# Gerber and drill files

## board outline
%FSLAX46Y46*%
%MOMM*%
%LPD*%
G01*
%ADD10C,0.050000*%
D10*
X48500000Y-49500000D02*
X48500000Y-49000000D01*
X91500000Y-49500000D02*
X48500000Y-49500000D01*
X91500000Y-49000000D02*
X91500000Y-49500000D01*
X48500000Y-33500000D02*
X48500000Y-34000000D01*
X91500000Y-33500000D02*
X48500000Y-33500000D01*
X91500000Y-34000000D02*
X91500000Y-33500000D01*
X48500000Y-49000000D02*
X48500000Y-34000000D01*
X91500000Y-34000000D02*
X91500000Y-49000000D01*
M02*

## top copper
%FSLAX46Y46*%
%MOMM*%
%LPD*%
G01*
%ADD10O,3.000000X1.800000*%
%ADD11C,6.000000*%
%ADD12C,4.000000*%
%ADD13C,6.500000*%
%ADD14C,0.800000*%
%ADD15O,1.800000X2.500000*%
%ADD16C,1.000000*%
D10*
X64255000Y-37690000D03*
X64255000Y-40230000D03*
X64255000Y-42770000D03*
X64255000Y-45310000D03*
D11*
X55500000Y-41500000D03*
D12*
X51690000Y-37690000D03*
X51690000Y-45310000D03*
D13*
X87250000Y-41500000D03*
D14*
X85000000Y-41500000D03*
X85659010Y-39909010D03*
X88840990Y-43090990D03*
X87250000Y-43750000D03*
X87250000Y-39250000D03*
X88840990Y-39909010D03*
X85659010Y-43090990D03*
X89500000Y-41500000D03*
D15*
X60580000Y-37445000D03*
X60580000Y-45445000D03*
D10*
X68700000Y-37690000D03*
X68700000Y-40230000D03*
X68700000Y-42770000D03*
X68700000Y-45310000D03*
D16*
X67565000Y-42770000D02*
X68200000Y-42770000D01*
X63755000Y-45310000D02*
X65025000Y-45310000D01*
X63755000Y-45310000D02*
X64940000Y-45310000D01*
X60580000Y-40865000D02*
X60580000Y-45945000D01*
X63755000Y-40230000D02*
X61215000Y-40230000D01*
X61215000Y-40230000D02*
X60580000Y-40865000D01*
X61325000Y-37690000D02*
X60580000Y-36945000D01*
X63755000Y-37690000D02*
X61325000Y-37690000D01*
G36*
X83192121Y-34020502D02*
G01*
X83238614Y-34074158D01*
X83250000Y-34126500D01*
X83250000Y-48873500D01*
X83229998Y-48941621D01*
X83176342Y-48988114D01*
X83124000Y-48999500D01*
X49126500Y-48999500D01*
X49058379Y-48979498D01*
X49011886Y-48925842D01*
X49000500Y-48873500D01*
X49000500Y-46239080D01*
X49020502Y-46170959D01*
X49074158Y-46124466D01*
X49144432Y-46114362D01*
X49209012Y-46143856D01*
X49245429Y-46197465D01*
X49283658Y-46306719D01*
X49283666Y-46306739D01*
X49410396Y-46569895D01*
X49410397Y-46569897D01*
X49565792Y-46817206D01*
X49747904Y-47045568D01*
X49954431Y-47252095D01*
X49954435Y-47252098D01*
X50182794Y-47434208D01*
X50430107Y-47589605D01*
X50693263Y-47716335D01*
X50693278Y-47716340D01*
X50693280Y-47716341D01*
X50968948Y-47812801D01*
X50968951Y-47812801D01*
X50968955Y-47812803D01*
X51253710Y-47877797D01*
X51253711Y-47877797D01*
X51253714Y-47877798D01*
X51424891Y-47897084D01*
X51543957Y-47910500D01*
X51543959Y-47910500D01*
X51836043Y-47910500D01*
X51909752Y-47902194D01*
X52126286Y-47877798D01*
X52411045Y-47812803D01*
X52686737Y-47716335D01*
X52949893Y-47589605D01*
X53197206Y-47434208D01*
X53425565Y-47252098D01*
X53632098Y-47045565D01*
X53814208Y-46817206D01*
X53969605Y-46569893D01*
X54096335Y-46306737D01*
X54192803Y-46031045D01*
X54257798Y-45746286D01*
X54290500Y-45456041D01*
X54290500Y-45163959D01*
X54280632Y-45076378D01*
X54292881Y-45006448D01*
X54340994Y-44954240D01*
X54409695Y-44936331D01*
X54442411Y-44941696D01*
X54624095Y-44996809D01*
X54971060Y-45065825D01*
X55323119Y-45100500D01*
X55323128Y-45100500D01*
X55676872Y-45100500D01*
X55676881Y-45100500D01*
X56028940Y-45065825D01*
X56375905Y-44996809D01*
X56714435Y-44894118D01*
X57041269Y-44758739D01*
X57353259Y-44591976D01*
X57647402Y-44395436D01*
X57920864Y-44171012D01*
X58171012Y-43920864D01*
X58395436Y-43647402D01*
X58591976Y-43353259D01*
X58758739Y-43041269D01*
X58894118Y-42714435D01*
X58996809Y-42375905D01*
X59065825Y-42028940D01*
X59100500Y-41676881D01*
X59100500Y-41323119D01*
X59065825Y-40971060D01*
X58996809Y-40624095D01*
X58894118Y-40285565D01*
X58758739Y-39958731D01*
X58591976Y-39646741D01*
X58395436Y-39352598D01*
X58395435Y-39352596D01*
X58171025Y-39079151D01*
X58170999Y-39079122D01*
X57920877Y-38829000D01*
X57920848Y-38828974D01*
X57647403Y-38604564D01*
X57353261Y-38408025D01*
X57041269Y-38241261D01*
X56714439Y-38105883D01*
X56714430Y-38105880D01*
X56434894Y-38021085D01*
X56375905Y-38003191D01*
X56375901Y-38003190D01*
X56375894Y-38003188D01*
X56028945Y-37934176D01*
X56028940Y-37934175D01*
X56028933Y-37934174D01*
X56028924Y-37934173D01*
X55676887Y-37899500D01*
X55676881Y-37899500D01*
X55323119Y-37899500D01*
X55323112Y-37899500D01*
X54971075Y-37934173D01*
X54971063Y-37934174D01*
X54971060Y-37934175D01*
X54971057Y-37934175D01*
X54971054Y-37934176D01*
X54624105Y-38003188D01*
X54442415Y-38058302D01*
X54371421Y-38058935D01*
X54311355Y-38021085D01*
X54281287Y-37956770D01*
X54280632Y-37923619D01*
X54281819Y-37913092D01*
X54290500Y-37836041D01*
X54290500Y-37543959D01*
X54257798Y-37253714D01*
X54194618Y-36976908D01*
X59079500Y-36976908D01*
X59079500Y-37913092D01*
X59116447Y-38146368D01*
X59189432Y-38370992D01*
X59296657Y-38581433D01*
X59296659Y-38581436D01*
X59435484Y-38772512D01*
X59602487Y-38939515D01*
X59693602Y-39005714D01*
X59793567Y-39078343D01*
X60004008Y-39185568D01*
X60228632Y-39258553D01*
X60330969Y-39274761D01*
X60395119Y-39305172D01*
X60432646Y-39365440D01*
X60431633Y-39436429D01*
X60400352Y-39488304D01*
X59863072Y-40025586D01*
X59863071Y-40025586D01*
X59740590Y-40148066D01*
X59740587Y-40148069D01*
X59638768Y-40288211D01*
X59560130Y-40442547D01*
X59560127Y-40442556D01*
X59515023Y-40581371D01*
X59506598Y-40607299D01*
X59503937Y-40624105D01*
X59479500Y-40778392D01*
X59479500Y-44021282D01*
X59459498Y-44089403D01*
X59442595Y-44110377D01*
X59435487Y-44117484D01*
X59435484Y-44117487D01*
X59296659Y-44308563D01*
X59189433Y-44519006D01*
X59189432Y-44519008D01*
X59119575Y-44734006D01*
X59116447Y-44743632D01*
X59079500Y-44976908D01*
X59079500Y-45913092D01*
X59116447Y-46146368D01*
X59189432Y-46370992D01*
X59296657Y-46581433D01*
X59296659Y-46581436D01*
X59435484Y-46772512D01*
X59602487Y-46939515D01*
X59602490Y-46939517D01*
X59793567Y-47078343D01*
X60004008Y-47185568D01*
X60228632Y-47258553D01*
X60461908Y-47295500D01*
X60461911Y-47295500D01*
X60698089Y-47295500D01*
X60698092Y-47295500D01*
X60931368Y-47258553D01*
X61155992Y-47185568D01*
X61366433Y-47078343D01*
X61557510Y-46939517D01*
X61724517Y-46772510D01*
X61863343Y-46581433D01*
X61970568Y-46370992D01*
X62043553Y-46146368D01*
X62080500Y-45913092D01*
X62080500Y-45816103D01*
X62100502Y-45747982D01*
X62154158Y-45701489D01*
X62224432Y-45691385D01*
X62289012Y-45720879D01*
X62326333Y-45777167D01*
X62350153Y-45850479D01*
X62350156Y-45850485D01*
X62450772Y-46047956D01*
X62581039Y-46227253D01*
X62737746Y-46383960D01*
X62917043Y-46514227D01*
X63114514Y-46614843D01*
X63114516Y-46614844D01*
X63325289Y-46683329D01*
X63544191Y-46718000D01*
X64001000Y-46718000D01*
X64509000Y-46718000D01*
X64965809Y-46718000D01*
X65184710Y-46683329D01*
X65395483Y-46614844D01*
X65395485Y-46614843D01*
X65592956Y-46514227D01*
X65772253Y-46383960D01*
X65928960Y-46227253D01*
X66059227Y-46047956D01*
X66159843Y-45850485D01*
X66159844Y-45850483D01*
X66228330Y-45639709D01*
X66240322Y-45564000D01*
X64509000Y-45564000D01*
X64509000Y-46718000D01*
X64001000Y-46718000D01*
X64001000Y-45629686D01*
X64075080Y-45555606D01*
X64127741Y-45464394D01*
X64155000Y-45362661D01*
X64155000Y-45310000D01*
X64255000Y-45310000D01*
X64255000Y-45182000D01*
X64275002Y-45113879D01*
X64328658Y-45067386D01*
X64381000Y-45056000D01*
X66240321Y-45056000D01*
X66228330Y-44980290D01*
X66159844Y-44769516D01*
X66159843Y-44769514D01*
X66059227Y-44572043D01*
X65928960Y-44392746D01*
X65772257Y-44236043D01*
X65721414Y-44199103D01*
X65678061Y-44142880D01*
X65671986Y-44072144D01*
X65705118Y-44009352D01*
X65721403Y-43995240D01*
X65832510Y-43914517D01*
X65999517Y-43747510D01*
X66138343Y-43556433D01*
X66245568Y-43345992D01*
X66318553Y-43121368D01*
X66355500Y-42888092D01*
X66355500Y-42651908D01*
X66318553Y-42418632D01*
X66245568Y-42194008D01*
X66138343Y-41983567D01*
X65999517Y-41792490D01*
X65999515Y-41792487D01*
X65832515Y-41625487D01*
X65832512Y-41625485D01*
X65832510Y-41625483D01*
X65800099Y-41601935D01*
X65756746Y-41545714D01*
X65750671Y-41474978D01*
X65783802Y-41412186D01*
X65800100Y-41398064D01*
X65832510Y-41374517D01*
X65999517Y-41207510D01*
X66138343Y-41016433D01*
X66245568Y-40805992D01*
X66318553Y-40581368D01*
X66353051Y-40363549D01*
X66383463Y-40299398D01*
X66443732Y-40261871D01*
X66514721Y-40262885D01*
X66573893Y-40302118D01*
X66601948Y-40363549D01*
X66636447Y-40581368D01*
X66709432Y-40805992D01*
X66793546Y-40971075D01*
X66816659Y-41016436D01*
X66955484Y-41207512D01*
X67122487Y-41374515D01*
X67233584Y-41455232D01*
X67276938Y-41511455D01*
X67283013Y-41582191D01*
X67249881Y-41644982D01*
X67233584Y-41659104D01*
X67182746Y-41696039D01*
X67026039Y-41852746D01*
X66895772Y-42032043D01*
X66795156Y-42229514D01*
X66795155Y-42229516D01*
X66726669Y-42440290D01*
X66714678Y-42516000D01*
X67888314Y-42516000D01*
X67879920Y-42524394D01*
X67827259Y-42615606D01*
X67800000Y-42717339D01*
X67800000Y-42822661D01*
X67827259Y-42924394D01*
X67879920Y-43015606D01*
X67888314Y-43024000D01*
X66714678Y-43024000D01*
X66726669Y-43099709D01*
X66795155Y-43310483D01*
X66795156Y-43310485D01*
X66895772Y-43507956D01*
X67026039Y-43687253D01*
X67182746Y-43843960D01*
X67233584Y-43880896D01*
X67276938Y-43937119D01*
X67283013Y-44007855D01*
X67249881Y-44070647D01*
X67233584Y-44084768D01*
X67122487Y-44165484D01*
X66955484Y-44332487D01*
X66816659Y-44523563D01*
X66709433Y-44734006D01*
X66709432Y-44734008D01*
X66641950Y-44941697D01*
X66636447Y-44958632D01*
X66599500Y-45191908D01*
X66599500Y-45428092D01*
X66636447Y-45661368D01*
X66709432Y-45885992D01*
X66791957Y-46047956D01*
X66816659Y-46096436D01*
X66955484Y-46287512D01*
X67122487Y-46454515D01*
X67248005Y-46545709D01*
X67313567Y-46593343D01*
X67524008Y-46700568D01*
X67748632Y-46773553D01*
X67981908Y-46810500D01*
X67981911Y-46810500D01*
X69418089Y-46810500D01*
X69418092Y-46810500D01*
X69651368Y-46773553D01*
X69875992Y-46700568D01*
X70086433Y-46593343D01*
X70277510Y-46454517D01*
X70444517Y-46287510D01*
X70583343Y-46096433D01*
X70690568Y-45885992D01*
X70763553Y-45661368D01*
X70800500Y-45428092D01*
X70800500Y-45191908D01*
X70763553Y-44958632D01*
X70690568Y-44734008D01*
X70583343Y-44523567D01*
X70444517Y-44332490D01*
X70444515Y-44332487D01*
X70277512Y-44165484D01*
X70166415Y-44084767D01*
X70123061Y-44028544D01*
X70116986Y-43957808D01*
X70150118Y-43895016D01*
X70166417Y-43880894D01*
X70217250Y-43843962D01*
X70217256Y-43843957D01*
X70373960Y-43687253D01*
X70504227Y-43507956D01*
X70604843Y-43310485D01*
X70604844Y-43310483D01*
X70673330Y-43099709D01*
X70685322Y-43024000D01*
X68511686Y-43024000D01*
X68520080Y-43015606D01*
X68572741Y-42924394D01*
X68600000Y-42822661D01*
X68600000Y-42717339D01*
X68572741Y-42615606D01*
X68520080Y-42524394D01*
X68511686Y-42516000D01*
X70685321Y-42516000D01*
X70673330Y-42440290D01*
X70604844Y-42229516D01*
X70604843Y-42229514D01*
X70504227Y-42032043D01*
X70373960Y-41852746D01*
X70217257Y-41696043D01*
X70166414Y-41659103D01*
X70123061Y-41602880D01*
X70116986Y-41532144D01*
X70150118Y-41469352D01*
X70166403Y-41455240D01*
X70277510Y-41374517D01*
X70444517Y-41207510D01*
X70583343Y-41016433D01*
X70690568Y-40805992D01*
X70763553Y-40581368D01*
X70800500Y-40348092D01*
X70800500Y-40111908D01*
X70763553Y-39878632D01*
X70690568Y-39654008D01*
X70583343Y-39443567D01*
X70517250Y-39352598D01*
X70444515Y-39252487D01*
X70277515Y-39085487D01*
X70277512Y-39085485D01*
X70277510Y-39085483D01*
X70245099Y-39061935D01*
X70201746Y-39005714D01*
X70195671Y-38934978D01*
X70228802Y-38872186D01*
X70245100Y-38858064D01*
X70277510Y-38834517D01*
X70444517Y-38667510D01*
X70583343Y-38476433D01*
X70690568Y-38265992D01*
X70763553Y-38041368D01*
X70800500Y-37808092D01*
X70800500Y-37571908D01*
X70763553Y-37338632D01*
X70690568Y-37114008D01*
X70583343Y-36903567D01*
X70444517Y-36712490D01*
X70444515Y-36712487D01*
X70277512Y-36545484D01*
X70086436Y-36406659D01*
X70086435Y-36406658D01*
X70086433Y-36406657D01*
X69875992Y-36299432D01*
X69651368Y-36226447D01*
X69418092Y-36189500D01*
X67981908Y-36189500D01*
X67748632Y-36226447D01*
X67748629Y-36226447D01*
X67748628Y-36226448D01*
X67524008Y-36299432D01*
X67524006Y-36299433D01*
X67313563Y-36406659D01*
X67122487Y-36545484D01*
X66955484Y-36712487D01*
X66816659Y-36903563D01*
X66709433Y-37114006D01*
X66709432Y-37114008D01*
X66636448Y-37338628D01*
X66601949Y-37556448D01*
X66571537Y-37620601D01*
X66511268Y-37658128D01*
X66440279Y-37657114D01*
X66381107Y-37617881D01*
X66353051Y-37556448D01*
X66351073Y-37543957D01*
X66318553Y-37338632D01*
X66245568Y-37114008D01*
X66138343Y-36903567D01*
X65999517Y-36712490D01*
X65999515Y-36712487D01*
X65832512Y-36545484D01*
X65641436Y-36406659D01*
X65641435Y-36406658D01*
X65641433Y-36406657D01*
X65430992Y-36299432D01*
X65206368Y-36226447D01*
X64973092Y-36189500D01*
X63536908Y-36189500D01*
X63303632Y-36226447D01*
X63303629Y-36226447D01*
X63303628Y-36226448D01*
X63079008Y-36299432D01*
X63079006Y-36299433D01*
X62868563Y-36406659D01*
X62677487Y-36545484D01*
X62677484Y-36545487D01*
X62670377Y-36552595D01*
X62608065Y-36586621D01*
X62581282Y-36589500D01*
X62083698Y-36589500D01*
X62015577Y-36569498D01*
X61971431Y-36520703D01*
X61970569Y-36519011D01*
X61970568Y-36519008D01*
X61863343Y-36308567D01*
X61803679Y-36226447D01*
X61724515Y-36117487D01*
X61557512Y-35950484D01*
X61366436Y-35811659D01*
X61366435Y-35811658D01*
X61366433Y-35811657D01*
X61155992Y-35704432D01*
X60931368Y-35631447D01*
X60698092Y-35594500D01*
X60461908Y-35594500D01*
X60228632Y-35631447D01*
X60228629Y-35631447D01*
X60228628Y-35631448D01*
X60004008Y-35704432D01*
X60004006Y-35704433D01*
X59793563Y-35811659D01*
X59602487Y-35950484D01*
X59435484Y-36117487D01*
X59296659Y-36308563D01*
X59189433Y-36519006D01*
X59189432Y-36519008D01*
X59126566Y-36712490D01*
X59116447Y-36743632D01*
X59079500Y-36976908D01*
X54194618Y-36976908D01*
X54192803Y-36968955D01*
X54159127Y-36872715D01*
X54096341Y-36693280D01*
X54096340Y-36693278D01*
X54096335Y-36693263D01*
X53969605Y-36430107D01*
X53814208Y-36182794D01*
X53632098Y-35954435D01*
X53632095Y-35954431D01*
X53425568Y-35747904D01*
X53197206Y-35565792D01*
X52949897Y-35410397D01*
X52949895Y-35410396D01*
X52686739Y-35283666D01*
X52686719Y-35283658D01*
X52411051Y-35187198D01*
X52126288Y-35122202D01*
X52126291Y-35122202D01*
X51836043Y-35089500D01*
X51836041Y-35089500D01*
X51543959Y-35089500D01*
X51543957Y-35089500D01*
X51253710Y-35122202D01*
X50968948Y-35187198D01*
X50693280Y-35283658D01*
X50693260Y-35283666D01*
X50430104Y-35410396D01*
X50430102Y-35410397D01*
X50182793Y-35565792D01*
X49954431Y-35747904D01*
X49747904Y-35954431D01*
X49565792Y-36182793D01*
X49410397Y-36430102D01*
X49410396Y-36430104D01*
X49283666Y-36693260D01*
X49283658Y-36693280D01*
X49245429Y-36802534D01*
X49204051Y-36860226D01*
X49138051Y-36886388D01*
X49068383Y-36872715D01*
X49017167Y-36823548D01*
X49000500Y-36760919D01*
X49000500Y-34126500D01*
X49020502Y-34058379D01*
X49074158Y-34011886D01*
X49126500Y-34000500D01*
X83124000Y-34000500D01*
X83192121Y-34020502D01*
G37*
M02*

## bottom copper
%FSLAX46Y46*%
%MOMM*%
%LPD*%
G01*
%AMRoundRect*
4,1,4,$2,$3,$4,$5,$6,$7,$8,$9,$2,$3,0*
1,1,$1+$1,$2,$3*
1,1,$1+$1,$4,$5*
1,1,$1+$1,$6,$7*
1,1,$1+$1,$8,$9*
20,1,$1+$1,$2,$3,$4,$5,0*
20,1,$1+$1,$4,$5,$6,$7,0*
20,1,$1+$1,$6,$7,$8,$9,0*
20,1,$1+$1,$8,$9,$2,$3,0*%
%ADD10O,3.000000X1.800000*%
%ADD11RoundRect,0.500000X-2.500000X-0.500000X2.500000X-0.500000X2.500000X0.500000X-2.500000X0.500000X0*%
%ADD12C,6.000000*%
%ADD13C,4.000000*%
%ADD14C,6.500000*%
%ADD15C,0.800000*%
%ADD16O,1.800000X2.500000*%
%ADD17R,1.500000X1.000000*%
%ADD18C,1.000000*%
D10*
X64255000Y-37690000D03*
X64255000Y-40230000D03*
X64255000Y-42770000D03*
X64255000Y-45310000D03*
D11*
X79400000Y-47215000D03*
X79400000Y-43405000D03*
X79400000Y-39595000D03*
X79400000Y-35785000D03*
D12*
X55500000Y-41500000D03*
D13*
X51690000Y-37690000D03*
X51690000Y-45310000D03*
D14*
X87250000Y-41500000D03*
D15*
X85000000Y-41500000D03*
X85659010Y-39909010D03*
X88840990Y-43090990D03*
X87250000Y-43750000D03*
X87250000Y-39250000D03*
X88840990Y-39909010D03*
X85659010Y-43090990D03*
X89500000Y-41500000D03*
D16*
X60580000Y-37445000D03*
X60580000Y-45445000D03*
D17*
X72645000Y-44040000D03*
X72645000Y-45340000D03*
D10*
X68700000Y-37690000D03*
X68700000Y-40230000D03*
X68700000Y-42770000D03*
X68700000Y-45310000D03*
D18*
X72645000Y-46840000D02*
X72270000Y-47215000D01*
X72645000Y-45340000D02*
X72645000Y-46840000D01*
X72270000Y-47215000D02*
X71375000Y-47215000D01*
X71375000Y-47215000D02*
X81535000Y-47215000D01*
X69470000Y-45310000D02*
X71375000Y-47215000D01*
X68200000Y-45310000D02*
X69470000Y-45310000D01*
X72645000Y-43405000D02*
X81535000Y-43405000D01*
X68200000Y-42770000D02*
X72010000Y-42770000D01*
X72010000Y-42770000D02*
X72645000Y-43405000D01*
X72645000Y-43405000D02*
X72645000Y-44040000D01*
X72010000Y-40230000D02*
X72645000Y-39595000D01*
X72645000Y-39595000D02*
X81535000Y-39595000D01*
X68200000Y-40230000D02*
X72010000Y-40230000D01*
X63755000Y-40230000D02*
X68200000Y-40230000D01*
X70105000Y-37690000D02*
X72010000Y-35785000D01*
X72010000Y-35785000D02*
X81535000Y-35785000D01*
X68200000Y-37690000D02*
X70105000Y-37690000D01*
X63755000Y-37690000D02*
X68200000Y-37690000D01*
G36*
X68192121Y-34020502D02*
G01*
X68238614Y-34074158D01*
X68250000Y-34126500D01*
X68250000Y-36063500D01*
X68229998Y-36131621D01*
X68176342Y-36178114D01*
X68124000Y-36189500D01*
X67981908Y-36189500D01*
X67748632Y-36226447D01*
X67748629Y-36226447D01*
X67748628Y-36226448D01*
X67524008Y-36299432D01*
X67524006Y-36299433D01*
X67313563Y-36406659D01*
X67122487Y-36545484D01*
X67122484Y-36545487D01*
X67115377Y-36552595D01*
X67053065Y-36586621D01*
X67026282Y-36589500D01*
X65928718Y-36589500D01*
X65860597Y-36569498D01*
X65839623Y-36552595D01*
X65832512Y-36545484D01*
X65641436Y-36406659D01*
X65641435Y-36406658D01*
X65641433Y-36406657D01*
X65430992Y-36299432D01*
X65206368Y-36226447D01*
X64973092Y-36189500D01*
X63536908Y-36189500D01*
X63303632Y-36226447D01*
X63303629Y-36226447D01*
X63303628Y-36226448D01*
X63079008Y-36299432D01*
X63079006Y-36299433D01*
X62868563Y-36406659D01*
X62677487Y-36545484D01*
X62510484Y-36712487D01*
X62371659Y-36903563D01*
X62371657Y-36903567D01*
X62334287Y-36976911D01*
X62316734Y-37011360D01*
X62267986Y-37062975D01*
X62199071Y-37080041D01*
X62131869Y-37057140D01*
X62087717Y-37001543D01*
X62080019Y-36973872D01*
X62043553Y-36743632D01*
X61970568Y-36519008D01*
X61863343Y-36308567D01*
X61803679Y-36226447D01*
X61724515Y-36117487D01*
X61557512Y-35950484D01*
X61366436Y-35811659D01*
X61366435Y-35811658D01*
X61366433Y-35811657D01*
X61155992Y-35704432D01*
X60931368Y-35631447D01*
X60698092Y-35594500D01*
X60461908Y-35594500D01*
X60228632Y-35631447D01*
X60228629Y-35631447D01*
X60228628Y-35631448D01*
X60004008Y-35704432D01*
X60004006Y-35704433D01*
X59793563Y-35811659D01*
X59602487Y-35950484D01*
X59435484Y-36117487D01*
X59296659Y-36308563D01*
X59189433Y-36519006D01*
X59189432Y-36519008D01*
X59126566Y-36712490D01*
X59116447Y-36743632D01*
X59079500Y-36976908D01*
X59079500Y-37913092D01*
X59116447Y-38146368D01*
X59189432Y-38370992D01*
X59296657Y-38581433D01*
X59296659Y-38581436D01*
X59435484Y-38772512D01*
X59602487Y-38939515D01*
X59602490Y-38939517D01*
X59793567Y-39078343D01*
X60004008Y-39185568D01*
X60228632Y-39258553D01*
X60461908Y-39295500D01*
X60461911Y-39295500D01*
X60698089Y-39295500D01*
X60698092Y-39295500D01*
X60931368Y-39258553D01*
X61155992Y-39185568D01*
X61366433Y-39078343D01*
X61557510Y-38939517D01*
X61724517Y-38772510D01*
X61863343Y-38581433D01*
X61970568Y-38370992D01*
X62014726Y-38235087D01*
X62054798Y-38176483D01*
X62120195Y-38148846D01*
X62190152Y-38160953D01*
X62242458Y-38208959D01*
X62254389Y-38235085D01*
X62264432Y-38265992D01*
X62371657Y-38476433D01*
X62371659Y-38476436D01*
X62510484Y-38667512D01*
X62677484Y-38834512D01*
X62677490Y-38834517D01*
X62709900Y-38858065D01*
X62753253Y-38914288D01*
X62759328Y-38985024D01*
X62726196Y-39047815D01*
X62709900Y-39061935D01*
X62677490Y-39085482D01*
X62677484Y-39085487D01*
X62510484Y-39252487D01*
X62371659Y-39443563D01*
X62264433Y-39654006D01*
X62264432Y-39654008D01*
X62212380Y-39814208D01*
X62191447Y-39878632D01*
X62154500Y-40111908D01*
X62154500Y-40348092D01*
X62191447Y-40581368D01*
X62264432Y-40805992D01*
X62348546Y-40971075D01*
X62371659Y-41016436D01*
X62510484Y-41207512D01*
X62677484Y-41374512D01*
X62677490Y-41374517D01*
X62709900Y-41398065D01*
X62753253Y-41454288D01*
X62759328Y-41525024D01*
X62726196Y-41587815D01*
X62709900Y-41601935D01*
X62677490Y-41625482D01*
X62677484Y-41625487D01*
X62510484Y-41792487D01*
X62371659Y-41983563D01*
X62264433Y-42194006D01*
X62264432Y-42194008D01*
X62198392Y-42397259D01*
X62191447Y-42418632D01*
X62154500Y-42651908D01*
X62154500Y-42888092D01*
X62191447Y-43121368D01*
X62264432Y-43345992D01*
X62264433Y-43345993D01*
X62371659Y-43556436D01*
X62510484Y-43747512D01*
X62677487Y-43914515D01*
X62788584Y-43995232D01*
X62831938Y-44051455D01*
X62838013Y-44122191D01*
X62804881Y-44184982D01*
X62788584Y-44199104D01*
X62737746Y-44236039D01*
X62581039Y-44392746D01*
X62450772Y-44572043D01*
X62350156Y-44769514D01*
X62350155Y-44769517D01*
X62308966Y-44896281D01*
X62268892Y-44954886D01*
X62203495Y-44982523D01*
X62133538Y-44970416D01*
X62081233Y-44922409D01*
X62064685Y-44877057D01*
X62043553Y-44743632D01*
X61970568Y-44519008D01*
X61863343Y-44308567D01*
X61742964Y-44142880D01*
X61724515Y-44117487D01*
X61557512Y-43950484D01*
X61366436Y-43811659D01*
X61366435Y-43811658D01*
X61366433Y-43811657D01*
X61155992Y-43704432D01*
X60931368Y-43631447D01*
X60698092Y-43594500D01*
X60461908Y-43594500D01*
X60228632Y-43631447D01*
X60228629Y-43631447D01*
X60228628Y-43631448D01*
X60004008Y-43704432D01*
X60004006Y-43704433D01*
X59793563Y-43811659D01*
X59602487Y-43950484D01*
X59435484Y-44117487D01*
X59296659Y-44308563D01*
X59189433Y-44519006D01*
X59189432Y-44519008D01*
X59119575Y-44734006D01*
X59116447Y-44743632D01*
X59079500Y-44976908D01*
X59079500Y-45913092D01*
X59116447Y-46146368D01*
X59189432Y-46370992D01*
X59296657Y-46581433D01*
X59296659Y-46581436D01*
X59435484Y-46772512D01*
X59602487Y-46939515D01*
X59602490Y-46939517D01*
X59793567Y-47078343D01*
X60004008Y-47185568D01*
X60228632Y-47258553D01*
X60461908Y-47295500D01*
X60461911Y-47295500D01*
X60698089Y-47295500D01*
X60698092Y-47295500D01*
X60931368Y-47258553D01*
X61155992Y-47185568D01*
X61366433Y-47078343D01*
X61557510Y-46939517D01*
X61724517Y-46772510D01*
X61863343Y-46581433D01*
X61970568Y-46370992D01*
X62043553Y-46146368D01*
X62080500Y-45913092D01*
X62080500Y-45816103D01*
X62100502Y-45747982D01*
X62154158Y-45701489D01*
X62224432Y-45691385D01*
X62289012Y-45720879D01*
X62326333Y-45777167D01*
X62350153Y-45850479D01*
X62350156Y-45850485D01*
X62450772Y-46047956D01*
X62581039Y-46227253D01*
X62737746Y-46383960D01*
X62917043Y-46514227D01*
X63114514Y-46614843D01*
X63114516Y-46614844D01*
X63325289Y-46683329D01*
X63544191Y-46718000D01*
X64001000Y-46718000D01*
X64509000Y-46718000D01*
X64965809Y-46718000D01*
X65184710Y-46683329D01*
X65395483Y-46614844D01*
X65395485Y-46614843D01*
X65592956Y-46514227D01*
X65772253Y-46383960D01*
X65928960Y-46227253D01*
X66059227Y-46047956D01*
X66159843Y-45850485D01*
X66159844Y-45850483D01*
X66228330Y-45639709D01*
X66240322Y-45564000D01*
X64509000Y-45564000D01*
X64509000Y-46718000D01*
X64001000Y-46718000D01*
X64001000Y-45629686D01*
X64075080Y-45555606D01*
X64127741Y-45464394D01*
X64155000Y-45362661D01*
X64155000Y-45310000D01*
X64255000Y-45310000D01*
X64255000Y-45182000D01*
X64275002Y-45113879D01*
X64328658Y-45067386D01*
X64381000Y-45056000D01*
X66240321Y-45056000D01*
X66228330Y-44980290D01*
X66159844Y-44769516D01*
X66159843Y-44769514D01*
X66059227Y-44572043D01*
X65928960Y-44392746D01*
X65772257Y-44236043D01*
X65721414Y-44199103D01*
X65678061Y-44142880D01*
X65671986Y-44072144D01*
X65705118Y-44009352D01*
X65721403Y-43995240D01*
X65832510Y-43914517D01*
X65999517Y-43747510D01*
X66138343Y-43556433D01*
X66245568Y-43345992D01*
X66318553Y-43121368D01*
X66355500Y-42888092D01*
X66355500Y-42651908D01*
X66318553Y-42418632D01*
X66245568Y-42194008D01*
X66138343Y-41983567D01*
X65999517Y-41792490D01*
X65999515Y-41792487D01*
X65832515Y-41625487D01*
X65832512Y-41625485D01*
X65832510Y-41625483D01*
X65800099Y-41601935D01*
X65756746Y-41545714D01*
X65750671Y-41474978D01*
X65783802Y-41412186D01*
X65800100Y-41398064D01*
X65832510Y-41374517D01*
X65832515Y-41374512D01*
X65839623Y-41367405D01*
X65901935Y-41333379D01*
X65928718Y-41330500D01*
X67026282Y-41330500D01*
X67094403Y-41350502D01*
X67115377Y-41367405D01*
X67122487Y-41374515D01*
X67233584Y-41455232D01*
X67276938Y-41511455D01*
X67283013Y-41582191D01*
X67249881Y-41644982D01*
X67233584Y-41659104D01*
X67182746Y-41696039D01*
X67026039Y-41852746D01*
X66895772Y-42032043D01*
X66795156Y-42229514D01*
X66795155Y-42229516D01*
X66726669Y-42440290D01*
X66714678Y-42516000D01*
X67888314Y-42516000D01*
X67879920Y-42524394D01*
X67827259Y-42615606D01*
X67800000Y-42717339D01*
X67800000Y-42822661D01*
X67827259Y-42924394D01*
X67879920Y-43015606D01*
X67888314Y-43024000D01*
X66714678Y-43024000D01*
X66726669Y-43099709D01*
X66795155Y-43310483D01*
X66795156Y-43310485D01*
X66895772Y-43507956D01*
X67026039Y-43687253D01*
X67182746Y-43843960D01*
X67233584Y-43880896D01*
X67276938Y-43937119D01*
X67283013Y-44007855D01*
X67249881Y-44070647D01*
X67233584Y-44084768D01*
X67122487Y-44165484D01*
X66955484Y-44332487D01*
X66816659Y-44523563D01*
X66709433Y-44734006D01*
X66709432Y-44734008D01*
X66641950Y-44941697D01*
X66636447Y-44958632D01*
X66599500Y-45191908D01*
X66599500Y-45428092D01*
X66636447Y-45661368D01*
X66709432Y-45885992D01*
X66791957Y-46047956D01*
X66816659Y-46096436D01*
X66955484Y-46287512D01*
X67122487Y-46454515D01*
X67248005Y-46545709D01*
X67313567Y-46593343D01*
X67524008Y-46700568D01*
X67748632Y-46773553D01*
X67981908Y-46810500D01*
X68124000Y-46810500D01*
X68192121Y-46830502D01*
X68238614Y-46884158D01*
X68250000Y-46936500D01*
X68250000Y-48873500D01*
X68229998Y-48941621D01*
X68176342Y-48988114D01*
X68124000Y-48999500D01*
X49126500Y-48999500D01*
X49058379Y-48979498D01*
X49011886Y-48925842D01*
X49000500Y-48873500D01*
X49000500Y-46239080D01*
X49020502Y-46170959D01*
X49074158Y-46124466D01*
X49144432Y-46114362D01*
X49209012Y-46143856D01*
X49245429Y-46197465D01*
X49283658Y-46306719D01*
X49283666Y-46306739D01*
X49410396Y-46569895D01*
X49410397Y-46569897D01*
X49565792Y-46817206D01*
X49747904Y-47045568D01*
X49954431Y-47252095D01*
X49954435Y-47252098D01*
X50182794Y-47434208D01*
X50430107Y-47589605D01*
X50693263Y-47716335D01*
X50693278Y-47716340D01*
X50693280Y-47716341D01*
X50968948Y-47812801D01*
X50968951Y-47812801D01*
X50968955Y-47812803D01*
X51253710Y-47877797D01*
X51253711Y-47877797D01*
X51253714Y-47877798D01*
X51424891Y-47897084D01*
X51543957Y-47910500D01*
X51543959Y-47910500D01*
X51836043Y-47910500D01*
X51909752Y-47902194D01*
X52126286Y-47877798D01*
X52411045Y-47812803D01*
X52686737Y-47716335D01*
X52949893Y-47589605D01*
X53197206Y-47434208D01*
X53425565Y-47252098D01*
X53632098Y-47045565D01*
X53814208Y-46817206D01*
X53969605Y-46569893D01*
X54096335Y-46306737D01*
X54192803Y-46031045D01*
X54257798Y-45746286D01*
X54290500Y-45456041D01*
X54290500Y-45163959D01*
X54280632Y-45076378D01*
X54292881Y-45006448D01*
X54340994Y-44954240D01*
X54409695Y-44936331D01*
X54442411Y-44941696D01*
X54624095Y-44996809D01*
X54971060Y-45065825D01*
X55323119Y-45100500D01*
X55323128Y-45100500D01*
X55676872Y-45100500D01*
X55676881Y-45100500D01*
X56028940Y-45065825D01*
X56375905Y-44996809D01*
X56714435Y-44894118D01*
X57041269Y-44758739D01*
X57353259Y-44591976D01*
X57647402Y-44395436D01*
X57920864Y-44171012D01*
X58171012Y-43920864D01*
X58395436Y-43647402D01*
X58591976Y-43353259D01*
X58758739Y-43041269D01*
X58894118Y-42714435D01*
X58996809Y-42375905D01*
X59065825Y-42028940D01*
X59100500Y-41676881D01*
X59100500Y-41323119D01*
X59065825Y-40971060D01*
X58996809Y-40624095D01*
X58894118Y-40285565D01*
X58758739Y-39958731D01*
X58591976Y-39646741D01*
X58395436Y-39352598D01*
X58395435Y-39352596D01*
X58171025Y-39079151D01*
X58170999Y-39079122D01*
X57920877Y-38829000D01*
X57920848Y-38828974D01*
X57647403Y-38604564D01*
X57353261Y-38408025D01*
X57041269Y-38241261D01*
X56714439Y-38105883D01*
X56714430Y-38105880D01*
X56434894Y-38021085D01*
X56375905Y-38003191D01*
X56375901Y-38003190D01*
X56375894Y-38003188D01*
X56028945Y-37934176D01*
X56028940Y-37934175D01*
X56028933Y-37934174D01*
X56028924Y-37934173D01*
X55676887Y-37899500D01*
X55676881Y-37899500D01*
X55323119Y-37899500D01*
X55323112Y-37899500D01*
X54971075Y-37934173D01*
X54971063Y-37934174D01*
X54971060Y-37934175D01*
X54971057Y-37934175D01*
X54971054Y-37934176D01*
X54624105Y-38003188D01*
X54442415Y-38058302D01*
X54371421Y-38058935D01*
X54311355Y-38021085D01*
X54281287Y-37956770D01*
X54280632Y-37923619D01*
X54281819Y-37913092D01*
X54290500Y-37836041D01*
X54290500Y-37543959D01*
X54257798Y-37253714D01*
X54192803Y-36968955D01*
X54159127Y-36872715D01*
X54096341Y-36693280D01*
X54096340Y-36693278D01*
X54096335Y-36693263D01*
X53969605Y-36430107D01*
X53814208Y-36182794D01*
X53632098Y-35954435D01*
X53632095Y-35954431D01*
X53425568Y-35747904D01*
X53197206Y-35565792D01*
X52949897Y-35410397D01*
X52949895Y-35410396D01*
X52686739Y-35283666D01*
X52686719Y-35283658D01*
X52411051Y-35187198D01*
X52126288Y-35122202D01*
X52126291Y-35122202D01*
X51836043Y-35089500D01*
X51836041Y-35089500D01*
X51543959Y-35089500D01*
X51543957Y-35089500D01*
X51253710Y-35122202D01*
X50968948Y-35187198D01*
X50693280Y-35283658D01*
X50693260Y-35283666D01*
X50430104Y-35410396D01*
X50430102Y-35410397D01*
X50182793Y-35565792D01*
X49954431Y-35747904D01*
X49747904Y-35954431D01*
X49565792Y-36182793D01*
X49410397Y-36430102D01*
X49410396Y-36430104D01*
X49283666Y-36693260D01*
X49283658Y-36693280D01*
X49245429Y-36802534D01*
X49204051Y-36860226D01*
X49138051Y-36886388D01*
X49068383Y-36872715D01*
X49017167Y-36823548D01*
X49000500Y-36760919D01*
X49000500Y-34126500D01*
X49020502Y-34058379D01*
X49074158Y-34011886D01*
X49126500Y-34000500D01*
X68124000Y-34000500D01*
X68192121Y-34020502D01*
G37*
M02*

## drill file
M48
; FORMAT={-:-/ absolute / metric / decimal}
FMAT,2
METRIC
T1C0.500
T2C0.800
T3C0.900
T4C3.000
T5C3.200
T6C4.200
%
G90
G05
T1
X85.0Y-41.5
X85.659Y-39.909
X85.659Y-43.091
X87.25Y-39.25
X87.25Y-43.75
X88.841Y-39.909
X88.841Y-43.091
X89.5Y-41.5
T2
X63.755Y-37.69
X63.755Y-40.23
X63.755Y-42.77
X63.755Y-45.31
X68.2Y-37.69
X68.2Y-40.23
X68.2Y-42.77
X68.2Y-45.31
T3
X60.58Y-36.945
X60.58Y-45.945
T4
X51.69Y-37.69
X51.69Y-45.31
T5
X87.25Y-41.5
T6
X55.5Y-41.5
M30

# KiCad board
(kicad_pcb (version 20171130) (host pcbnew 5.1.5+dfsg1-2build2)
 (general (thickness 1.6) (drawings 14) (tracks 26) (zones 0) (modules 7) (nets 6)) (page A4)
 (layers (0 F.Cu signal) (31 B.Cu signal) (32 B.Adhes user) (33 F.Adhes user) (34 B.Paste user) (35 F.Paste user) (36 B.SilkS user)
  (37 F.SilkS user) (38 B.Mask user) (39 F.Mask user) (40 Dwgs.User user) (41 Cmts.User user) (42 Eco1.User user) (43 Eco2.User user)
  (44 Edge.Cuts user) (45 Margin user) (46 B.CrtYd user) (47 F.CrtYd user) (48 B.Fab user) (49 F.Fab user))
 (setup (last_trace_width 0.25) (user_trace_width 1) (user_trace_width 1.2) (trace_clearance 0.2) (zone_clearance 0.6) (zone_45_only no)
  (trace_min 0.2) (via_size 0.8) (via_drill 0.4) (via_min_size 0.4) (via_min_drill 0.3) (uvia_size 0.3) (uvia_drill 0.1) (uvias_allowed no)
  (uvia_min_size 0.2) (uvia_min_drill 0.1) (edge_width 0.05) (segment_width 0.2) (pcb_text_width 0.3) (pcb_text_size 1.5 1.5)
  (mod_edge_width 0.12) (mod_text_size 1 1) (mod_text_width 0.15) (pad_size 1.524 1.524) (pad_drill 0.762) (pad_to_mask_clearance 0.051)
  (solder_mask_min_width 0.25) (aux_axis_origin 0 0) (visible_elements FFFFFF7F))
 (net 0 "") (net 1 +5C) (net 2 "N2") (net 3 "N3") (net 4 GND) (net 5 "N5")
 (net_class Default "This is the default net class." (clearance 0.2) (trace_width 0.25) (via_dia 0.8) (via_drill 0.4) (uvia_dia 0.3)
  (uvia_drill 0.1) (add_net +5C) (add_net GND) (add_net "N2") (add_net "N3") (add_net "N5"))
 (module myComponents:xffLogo (layer F.Cu) (at 79.375 41.275 270)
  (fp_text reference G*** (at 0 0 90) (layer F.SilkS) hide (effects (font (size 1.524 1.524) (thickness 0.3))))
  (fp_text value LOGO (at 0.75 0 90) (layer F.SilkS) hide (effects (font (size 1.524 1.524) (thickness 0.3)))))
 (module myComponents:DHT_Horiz (layer F.Cu) (at 63.755 37.69)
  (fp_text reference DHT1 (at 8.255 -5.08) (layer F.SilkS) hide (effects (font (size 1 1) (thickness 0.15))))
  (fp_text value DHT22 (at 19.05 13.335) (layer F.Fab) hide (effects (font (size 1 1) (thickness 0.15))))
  (pad 1 thru_hole oval (at 0 0) (size 3 1.8) (drill 0.8 (offset 0.5 0)) (layers *.Cu *.Mask) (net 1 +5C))
  (pad 2 thru_hole oval (at 0 2.54) (size 3 1.8) (drill 0.8 (offset 0.5 0)) (layers *.Cu *.Mask) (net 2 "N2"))
  (pad 3 thru_hole oval (at 0 5.08) (size 3 1.8) (drill 0.8 (offset 0.5 0)) (layers *.Cu *.Mask) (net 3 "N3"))
  (pad 4 thru_hole oval (at 0 7.62) (size 3 1.8) (drill 0.8 (offset 0.5 0)) (layers *.Cu *.Mask) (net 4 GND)))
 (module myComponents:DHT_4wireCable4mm (layer F.Cu) (at 55.5 41.5)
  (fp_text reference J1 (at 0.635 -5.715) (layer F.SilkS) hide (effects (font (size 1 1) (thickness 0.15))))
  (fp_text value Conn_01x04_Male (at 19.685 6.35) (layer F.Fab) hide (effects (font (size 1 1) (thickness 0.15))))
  (pad 4 smd roundrect (at 25.4 5.715) (size 6 2) (drill (offset -1.5 0)) (layers B.Cu B.Paste B.Mask) (roundrect_rratio 0.25) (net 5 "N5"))
  (pad 3 smd roundrect (at 25.4 1.905) (size 6 2) (drill (offset -1.5 0)) (layers B.Cu B.Paste B.Mask) (roundrect_rratio 0.25) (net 4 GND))
  (pad 2 smd roundrect (at 25.4 -1.905) (size 6 2) (drill (offset -1.5 0)) (layers B.Cu B.Paste B.Mask) (roundrect_rratio 0.25) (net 2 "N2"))
  (pad 1 smd roundrect (at 25.4 -5.715) (size 6 2) (drill (offset -1.5 0)) (layers B.Cu B.Paste B.Mask) (roundrect_rratio 0.25) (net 1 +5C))
  (pad "" thru_hole circle (at 0 0) (size 6 6) (drill 4.2) (layers *.Cu *.Mask))
  (pad "" thru_hole circle (at -3.81 -3.81) (size 4 4) (drill 3) (layers *.Cu *.Mask))
  (pad "" thru_hole circle (at -3.81 3.81) (size 4 4) (drill 3) (layers *.Cu *.Mask)))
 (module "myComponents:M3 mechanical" (layer F.Cu) (at 87.25 41.5)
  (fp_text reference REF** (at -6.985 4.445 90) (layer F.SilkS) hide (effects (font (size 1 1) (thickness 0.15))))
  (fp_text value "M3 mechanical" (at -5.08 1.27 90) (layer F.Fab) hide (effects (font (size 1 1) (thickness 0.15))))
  (pad "" thru_hole circle (at 0 0) (size 6.5 6.5) (drill 3.2) (layers *.Cu *.Mask))
  (pad 1 thru_hole circle (at -2.25 0) (size 0.8 0.8) (drill 0.5) (layers *.Cu *.Mask))
  (pad 1 thru_hole circle (at -1.59099 -1.59099) (size 0.8 0.8) (drill 0.5) (layers *.Cu *.Mask))
  (pad 1 thru_hole circle (at 1.59099 1.59099) (size 0.8 0.8) (drill 0.5) (layers *.Cu *.Mask))
  (pad 1 thru_hole circle (at 0 2.25) (size 0.8 0.8) (drill 0.5) (layers *.Cu *.Mask))
  (pad 1 thru_hole circle (at 0 -2.25) (size 0.8 0.8) (drill 0.5) (layers *.Cu *.Mask))
  (pad 1 thru_hole circle (at 1.59099 -1.59099) (size 0.8 0.8) (drill 0.5) (layers *.Cu *.Mask))
  (pad 1 thru_hole circle (at -1.59099 1.59099) (size 0.8 0.8) (drill 0.5) (layers *.Cu *.Mask))
  (pad 1 thru_hole circle (at 2.25 0) (size 0.8 0.8) (drill 0.5) (layers *.Cu *.Mask)))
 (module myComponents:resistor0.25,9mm (layer F.Cu) (at 60.58 36.945 270)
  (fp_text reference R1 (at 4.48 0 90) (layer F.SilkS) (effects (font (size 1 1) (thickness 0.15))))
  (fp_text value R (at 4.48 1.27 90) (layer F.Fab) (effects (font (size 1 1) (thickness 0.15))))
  (pad 1 thru_hole oval (at 0 0 270) (size 2.5 1.8) (drill 0.9 (offset 0.5 0)) (layers *.Cu *.Mask) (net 1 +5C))
  (pad 2 thru_hole oval (at 9 0 270) (size 2.5 1.8) (drill 0.9 (offset -0.5 0)) (layers *.Cu *.Mask) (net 2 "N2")))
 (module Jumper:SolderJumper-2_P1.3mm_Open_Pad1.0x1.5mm (layer B.Cu) (at 72.645 44.69 90)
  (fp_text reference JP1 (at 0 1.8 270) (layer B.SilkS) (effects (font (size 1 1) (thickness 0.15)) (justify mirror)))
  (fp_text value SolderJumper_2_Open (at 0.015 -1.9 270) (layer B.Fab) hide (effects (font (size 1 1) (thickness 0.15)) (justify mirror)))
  (pad 2 smd rect (at 0.65 0 90) (size 1 1.5) (layers B.Cu B.Mask) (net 4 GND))
  (pad 1 smd rect (at -0.65 0 90) (size 1 1.5) (layers B.Cu B.Mask) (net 5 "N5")))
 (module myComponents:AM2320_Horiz (layer F.Cu) (at 68.2 37.69)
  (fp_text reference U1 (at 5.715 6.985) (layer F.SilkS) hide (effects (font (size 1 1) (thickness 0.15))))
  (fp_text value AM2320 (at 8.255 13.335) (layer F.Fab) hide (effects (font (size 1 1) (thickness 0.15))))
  (pad 1 thru_hole oval (at 0 0) (size 3 1.8) (drill 0.8 (offset 0.5 0)) (layers *.Cu *.Mask) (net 1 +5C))
  (pad 2 thru_hole oval (at 0 2.54) (size 3 1.8) (drill 0.8 (offset 0.5 0)) (layers *.Cu *.Mask) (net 2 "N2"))
  (pad 3 thru_hole oval (at 0 5.08) (size 3 1.8) (drill 0.8 (offset 0.5 0)) (layers *.Cu *.Mask) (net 4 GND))
  (pad 4 thru_hole oval (at 0 7.62) (size 3 1.8) (drill 0.8 (offset 0.5 0)) (layers *.Cu *.Mask) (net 5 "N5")))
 (gr_line (start 48.5 49.5) (end 48.5 49) (layer Edge.Cuts) (width 0.05))
 (gr_line (start 91.5 49.5) (end 48.5 49.5) (layer Edge.Cuts) (width 0.05))
 (gr_line (start 91.5 49) (end 91.5 49.5) (layer Edge.Cuts) (width 0.05))
 (gr_line (start 48.5 33.5) (end 48.5 34) (layer Edge.Cuts) (width 0.05))
 (gr_line (start 91.5 33.5) (end 48.5 33.5) (layer Edge.Cuts) (width 0.05))
 (gr_line (start 91.5 34) (end 91.5 33.5) (layer Edge.Cuts) (width 0.05))
 (gr_line (start 48.5 49) (end 48.5 34) (layer Edge.Cuts) (width 0.05))
 (gr_line (start 91.5 34) (end 91.5 49) (layer Edge.Cuts) (width 0.05))
 (segment (start 72.645 46.84) (end 72.27 47.215) (width 1) (layer B.Cu) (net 5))
 (segment (start 72.645 45.34) (end 72.645 46.84) (width 1) (layer B.Cu) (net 5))
 (segment (start 72.27 47.215) (end 71.375 47.215) (width 1) (layer B.Cu) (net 5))
 (segment (start 71.375 47.215) (end 81.535 47.215) (width 1) (layer B.Cu) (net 5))
 (segment (start 69.47 45.31) (end 71.375 47.215) (width 1) (layer B.Cu) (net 5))
 (segment (start 68.2 45.31) (end 69.47 45.31) (width 1) (layer B.Cu) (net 5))
 (segment (start 67.565 42.77) (end 68.2 42.77) (width 1) (layer F.Cu) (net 4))
 (segment (start 72.645 43.405) (end 81.535 43.405) (width 1) (layer B.Cu) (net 4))
 (segment (start 68.2 42.77) (end 72.01 42.77) (width 1) (layer B.Cu) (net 4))
 (segment (start 72.01 42.77) (end 72.645 43.405) (width 1) (layer B.Cu) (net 4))
 (segment (start 72.645 43.405) (end 72.645 44.04) (width 1) (layer B.Cu) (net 4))
 (segment (start 63.755 45.31) (end 65.025 45.31) (width 1) (layer F.Cu) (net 4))
 (segment (start 63.755 45.31) (end 64.94 45.31) (width 1) (layer F.Cu) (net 4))
 (segment (start 72.01 40.23) (end 72.645 39.595) (width 1) (layer B.Cu) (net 2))
 (segment (start 60.58 40.865) (end 60.58 45.945) (width 1) (layer F.Cu) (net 2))
 (segment (start 72.645 39.595) (end 81.535 39.595) (width 1) (layer B.Cu) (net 2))
 (segment (start 68.2 40.23) (end 72.01 40.23) (width 1) (layer B.Cu) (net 2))
 (segment (start 63.755 40.23) (end 61.215 40.23) (width 1) (layer F.Cu) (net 2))
 (segment (start 61.215 40.23) (end 60.58 40.865) (width 1) (layer F.Cu) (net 2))
 (segment (start 63.755 40.23) (end 68.2 40.23) (width 1) (layer B.Cu) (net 2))
 (segment (start 61.325 37.69) (end 60.58 36.945) (width 1) (layer F.Cu) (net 1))
 (segment (start 63.755 37.69) (end 61.325 37.69) (width 1) (layer F.Cu) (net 1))
 (segment (start 70.105 37.69) (end 72.01 35.785) (width 1) (layer B.Cu) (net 1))
 (segment (start 72.01 35.785) (end 81.535 35.785) (width 1) (layer B.Cu) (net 1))
 (segment (start 68.2 37.69) (end 70.105 37.69) (width 1) (layer B.Cu) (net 1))
 (segment (start 63.755 37.69) (end 68.2 37.69) (width 1) (layer B.Cu) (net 1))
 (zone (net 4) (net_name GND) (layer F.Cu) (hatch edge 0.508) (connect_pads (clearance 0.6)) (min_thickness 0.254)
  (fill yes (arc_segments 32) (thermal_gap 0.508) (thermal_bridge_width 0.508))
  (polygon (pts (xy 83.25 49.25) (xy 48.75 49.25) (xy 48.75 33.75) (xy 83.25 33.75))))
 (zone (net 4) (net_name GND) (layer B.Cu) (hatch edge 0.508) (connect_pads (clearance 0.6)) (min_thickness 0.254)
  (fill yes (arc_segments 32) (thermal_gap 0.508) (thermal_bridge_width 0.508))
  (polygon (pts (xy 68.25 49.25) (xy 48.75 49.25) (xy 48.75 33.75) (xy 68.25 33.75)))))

